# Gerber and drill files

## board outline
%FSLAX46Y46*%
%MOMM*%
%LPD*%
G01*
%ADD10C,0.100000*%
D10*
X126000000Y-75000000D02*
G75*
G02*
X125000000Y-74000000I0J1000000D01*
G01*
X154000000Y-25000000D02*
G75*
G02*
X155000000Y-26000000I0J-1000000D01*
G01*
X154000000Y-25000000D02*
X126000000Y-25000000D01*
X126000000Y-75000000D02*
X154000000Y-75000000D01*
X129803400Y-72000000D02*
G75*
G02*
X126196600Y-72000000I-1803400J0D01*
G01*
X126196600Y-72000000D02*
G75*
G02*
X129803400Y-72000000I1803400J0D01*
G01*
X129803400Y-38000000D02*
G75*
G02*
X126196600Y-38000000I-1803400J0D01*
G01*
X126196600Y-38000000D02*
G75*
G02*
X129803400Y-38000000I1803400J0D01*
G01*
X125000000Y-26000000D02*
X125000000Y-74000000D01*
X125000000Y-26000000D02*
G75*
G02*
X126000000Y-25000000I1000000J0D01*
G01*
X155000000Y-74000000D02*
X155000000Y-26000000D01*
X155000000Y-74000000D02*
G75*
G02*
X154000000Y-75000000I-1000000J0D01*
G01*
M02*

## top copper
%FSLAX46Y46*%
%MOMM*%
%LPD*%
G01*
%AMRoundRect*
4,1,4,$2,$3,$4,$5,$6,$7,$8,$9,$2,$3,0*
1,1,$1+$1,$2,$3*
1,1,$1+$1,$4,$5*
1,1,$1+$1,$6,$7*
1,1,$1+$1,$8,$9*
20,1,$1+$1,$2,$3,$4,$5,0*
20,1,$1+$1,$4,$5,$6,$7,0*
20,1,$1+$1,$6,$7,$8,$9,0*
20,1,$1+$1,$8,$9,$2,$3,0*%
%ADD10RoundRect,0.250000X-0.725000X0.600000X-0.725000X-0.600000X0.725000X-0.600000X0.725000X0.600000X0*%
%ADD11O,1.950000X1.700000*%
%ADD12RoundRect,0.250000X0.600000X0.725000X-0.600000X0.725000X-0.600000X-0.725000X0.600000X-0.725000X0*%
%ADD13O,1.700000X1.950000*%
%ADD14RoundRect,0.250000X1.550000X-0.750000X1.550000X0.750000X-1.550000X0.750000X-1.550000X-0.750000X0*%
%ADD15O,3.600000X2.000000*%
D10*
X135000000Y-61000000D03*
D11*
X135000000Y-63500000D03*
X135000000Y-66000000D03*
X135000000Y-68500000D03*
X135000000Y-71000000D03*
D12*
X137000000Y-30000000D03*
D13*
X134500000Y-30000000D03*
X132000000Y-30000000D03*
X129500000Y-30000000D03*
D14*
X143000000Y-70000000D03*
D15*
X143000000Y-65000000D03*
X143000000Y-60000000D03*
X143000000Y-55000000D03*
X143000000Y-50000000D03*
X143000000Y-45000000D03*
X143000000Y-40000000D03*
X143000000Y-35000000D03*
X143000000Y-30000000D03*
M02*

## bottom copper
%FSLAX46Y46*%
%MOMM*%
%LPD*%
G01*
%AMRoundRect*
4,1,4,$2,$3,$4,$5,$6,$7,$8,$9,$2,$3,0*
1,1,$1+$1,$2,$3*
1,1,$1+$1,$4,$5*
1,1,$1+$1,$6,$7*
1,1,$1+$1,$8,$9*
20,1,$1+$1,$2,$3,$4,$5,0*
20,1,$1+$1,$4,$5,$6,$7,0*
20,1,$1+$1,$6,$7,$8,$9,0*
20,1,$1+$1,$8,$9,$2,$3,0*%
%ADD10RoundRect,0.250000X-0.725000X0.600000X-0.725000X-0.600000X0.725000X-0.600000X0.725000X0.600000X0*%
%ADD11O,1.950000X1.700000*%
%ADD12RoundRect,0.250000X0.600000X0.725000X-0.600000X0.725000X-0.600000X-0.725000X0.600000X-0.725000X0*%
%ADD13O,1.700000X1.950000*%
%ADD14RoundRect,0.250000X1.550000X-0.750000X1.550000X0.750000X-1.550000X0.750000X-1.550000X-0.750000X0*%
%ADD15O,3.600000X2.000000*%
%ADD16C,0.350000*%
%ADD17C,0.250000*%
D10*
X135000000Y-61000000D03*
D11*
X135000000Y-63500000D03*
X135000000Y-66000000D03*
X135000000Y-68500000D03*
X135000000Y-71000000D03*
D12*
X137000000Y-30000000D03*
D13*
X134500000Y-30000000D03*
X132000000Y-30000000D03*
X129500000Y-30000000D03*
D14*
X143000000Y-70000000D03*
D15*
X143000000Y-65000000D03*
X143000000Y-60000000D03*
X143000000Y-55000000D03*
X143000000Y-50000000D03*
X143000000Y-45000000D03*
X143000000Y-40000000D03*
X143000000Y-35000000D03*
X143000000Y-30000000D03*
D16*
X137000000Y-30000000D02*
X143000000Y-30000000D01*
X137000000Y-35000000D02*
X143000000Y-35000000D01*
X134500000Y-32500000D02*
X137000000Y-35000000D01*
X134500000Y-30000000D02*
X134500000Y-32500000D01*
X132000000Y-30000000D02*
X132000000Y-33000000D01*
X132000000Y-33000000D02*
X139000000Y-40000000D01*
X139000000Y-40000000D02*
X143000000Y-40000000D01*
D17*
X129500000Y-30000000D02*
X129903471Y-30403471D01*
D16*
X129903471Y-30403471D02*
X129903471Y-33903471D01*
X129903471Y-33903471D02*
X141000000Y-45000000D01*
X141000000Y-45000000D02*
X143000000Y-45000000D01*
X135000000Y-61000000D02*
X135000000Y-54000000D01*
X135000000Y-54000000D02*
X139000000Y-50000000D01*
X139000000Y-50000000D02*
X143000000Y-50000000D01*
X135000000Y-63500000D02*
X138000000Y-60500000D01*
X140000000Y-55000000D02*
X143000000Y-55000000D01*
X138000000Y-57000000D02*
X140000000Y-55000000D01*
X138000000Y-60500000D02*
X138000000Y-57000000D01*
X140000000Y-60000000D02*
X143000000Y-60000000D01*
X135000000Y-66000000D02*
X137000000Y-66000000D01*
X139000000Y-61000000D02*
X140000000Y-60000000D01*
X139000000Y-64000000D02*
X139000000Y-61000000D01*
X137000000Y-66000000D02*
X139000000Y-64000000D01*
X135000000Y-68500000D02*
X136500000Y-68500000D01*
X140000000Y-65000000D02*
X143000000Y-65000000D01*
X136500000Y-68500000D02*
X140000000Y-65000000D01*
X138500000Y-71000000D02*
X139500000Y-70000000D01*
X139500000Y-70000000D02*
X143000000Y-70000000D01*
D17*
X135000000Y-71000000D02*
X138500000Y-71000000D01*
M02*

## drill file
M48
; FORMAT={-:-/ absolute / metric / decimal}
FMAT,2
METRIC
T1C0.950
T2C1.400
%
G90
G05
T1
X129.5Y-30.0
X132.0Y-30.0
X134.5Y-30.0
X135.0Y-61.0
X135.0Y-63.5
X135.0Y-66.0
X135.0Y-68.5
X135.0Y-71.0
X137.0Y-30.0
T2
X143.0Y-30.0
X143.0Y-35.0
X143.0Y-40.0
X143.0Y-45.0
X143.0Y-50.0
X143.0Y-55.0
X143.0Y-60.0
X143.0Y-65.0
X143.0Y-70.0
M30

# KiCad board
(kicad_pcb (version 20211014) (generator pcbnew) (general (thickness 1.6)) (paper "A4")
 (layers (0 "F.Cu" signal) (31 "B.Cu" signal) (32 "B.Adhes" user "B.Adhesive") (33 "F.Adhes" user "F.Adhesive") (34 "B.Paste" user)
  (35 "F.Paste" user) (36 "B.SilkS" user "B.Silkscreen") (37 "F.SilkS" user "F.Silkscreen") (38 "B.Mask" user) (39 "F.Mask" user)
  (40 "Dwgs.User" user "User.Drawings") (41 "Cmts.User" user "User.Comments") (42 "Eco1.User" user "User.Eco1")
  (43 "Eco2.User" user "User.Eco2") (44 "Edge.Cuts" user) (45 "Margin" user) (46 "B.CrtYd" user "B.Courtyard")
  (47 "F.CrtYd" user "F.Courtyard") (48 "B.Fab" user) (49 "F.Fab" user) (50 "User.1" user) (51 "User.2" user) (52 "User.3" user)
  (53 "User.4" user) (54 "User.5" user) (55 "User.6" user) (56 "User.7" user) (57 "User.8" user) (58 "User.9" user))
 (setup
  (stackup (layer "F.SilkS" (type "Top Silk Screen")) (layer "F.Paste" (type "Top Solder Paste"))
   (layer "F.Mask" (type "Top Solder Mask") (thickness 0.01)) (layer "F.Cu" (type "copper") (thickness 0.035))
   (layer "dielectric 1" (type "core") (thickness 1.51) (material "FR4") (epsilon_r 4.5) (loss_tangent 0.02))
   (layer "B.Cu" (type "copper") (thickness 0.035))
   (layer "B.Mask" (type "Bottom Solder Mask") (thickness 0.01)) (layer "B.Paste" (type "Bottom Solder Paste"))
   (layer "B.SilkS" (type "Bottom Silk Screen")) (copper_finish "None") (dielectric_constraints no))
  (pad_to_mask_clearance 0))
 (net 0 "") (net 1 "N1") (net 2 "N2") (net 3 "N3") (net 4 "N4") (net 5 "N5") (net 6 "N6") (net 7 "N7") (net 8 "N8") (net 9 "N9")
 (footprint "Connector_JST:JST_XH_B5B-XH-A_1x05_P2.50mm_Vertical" (layer "F.Cu") (at 135 61 -90)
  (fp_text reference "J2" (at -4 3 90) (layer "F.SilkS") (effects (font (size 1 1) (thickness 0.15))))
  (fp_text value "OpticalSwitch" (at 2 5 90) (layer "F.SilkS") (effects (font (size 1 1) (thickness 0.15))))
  (pad "1" thru_hole roundrect (at 0 0 270) (size 1.7 1.95) (drill 0.95) (layers *.Cu *.Mask) (roundrect_rratio 0.147059) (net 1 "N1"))
  (pad "2" thru_hole oval (at 2.5 0 270) (size 1.7 1.95) (drill 0.95) (layers *.Cu *.Mask) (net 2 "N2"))
  (pad "3" thru_hole oval (at 5 0 270) (size 1.7 1.95) (drill 0.95) (layers *.Cu *.Mask) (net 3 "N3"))
  (pad "4" thru_hole oval (at 7.5 0 270) (size 1.7 1.95) (drill 0.95) (layers *.Cu *.Mask) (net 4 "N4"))
  (pad "5" thru_hole oval (at 10 0 270) (size 1.7 1.95) (drill 0.95) (layers *.Cu *.Mask) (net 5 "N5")))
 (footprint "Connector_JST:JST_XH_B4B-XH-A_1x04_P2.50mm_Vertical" (layer "F.Cu") (at 137 30 180)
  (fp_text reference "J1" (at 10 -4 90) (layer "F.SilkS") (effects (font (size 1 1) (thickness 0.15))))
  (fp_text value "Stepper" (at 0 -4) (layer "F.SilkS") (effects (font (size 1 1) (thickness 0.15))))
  (pad "1" thru_hole roundrect (at 0 0 180) (size 1.7 1.95) (drill 0.95) (layers *.Cu *.Mask) (roundrect_rratio 0.147059) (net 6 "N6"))
  (pad "2" thru_hole oval (at 2.5 0 180) (size 1.7 1.95) (drill 0.95) (layers *.Cu *.Mask) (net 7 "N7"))
  (pad "3" thru_hole oval (at 5 0 180) (size 1.7 1.95) (drill 0.95) (layers *.Cu *.Mask) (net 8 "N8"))
  (pad "4" thru_hole oval (at 7.5 0 180) (size 1.7 1.95) (drill 0.95) (layers *.Cu *.Mask) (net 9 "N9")))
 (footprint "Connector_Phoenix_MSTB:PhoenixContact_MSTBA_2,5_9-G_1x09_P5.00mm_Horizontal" (layer "F.Cu") (at 143 70 90)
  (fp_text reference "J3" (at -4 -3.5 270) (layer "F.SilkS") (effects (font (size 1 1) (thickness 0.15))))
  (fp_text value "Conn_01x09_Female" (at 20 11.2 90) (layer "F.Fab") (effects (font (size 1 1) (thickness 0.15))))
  (pad "1" thru_hole roundrect (at 0 0 90) (size 2 3.6) (drill 1.4) (layers *.Cu *.Mask) (roundrect_rratio 0.125) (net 5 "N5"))
  (pad "2" thru_hole oval (at 5 0 90) (size 2 3.6) (drill 1.4) (layers *.Cu *.Mask) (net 4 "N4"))
  (pad "3" thru_hole oval (at 10 0 90) (size 2 3.6) (drill 1.4) (layers *.Cu *.Mask) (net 3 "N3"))
  (pad "4" thru_hole oval (at 15 0 90) (size 2 3.6) (drill 1.4) (layers *.Cu *.Mask) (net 2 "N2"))
  (pad "5" thru_hole oval (at 20 0 90) (size 2 3.6) (drill 1.4) (layers *.Cu *.Mask) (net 1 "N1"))
  (pad "6" thru_hole oval (at 25 0 90) (size 2 3.6) (drill 1.4) (layers *.Cu *.Mask) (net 9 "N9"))
  (pad "7" thru_hole oval (at 30 0 90) (size 2 3.6) (drill 1.4) (layers *.Cu *.Mask) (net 8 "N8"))
  (pad "8" thru_hole oval (at 35 0 90) (size 2 3.6) (drill 1.4) (layers *.Cu *.Mask) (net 7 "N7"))
  (pad "9" thru_hole oval (at 40 0 90) (size 2 3.6) (drill 1.4) (layers *.Cu *.Mask) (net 6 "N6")))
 (gr_arc (start 126 75) (mid 125.292893 74.707107) (end 125 74) (layer "Edge.Cuts") (width 0.1))
 (gr_arc (start 154 25) (mid 154.707107 25.292893) (end 155 26) (layer "Edge.Cuts") (width 0.1))
 (gr_line (start 154 25) (end 126 25) (layer "Edge.Cuts") (width 0.1))
 (gr_line (start 126 75) (end 154 75) (layer "Edge.Cuts") (width 0.1))
 (gr_circle (center 128 72) (end 129.8034 72) (layer "Edge.Cuts") (width 0.1) (fill none))
 (gr_circle (center 128 38) (end 129.8034 38) (layer "Edge.Cuts") (width 0.1) (fill none))
 (gr_line (start 125 26) (end 125 74) (layer "Edge.Cuts") (width 0.1))
 (gr_arc (start 125 26) (mid 125.292893 25.292893) (end 126 25) (layer "Edge.Cuts") (width 0.1))
 (gr_line (start 155 74) (end 155 26) (layer "Edge.Cuts") (width 0.1))
 (gr_arc (start 155 74) (mid 154.707107 74.707107) (end 154 75) (layer "Edge.Cuts") (width 0.1))
 (segment (start 137 30) (end 143 30) (width 0.35) (layer "B.Cu") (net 6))
 (segment (start 137 35) (end 143 35) (width 0.35) (layer "B.Cu") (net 7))
 (segment (start 134.5 32.5) (end 137 35) (width 0.35) (layer "B.Cu") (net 7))
 (segment (start 134.5 30) (end 134.5 32.5) (width 0.35) (layer "B.Cu") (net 7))
 (segment (start 132 30) (end 132 33) (width 0.35) (layer "B.Cu") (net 8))
 (segment (start 132 33) (end 139 40) (width 0.35) (layer "B.Cu") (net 8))
 (segment (start 139 40) (end 143 40) (width 0.35) (layer "B.Cu") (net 8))
 (segment (start 129.5 30) (end 129.903471 30.403471) (width 0.25) (layer "B.Cu") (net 9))
 (segment (start 129.903471 30.403471) (end 129.903471 33.903471) (width 0.35) (layer "B.Cu") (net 9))
 (segment (start 129.903471 33.903471) (end 141 45) (width 0.35) (layer "B.Cu") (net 9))
 (segment (start 141 45) (end 143 45) (width 0.35) (layer "B.Cu") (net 9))
 (segment (start 135 61) (end 135 54) (width 0.35) (layer "B.Cu") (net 1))
 (segment (start 135 54) (end 139 50) (width 0.35) (layer "B.Cu") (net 1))
 (segment (start 139 50) (end 143 50) (width 0.35) (layer "B.Cu") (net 1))
 (segment (start 135 63.5) (end 138 60.5) (width 0.35) (layer "B.Cu") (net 2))
 (segment (start 140 55) (end 143 55) (width 0.35) (layer "B.Cu") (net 2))
 (segment (start 138 57) (end 140 55) (width 0.35) (layer "B.Cu") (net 2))
 (segment (start 138 60.5) (end 138 57) (width 0.35) (layer "B.Cu") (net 2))
 (segment (start 140 60) (end 143 60) (width 0.35) (layer "B.Cu") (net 3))
 (segment (start 135 66) (end 137 66) (width 0.35) (layer "B.Cu") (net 3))
 (segment (start 139 61) (end 140 60) (width 0.35) (layer "B.Cu") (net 3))
 (segment (start 139 64) (end 139 61) (width 0.35) (layer "B.Cu") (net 3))
 (segment (start 137 66) (end 139 64) (width 0.35) (layer "B.Cu") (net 3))
 (segment (start 135 68.5) (end 136.5 68.5) (width 0.35) (layer "B.Cu") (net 4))
 (segment (start 140 65) (end 143 65) (width 0.35) (layer "B.Cu") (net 4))
 (segment (start 136.5 68.5) (end 140 65) (width 0.35) (layer "B.Cu") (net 4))
 (segment (start 138.5 71) (end 139.5 70) (width 0.35) (layer "B.Cu") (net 5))
 (segment (start 139.5 70) (end 143 70) (width 0.35) (layer "B.Cu") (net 5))
 (segment (start 135 71) (end 138.5 71) (width 0.25) (layer "B.Cu") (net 5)))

